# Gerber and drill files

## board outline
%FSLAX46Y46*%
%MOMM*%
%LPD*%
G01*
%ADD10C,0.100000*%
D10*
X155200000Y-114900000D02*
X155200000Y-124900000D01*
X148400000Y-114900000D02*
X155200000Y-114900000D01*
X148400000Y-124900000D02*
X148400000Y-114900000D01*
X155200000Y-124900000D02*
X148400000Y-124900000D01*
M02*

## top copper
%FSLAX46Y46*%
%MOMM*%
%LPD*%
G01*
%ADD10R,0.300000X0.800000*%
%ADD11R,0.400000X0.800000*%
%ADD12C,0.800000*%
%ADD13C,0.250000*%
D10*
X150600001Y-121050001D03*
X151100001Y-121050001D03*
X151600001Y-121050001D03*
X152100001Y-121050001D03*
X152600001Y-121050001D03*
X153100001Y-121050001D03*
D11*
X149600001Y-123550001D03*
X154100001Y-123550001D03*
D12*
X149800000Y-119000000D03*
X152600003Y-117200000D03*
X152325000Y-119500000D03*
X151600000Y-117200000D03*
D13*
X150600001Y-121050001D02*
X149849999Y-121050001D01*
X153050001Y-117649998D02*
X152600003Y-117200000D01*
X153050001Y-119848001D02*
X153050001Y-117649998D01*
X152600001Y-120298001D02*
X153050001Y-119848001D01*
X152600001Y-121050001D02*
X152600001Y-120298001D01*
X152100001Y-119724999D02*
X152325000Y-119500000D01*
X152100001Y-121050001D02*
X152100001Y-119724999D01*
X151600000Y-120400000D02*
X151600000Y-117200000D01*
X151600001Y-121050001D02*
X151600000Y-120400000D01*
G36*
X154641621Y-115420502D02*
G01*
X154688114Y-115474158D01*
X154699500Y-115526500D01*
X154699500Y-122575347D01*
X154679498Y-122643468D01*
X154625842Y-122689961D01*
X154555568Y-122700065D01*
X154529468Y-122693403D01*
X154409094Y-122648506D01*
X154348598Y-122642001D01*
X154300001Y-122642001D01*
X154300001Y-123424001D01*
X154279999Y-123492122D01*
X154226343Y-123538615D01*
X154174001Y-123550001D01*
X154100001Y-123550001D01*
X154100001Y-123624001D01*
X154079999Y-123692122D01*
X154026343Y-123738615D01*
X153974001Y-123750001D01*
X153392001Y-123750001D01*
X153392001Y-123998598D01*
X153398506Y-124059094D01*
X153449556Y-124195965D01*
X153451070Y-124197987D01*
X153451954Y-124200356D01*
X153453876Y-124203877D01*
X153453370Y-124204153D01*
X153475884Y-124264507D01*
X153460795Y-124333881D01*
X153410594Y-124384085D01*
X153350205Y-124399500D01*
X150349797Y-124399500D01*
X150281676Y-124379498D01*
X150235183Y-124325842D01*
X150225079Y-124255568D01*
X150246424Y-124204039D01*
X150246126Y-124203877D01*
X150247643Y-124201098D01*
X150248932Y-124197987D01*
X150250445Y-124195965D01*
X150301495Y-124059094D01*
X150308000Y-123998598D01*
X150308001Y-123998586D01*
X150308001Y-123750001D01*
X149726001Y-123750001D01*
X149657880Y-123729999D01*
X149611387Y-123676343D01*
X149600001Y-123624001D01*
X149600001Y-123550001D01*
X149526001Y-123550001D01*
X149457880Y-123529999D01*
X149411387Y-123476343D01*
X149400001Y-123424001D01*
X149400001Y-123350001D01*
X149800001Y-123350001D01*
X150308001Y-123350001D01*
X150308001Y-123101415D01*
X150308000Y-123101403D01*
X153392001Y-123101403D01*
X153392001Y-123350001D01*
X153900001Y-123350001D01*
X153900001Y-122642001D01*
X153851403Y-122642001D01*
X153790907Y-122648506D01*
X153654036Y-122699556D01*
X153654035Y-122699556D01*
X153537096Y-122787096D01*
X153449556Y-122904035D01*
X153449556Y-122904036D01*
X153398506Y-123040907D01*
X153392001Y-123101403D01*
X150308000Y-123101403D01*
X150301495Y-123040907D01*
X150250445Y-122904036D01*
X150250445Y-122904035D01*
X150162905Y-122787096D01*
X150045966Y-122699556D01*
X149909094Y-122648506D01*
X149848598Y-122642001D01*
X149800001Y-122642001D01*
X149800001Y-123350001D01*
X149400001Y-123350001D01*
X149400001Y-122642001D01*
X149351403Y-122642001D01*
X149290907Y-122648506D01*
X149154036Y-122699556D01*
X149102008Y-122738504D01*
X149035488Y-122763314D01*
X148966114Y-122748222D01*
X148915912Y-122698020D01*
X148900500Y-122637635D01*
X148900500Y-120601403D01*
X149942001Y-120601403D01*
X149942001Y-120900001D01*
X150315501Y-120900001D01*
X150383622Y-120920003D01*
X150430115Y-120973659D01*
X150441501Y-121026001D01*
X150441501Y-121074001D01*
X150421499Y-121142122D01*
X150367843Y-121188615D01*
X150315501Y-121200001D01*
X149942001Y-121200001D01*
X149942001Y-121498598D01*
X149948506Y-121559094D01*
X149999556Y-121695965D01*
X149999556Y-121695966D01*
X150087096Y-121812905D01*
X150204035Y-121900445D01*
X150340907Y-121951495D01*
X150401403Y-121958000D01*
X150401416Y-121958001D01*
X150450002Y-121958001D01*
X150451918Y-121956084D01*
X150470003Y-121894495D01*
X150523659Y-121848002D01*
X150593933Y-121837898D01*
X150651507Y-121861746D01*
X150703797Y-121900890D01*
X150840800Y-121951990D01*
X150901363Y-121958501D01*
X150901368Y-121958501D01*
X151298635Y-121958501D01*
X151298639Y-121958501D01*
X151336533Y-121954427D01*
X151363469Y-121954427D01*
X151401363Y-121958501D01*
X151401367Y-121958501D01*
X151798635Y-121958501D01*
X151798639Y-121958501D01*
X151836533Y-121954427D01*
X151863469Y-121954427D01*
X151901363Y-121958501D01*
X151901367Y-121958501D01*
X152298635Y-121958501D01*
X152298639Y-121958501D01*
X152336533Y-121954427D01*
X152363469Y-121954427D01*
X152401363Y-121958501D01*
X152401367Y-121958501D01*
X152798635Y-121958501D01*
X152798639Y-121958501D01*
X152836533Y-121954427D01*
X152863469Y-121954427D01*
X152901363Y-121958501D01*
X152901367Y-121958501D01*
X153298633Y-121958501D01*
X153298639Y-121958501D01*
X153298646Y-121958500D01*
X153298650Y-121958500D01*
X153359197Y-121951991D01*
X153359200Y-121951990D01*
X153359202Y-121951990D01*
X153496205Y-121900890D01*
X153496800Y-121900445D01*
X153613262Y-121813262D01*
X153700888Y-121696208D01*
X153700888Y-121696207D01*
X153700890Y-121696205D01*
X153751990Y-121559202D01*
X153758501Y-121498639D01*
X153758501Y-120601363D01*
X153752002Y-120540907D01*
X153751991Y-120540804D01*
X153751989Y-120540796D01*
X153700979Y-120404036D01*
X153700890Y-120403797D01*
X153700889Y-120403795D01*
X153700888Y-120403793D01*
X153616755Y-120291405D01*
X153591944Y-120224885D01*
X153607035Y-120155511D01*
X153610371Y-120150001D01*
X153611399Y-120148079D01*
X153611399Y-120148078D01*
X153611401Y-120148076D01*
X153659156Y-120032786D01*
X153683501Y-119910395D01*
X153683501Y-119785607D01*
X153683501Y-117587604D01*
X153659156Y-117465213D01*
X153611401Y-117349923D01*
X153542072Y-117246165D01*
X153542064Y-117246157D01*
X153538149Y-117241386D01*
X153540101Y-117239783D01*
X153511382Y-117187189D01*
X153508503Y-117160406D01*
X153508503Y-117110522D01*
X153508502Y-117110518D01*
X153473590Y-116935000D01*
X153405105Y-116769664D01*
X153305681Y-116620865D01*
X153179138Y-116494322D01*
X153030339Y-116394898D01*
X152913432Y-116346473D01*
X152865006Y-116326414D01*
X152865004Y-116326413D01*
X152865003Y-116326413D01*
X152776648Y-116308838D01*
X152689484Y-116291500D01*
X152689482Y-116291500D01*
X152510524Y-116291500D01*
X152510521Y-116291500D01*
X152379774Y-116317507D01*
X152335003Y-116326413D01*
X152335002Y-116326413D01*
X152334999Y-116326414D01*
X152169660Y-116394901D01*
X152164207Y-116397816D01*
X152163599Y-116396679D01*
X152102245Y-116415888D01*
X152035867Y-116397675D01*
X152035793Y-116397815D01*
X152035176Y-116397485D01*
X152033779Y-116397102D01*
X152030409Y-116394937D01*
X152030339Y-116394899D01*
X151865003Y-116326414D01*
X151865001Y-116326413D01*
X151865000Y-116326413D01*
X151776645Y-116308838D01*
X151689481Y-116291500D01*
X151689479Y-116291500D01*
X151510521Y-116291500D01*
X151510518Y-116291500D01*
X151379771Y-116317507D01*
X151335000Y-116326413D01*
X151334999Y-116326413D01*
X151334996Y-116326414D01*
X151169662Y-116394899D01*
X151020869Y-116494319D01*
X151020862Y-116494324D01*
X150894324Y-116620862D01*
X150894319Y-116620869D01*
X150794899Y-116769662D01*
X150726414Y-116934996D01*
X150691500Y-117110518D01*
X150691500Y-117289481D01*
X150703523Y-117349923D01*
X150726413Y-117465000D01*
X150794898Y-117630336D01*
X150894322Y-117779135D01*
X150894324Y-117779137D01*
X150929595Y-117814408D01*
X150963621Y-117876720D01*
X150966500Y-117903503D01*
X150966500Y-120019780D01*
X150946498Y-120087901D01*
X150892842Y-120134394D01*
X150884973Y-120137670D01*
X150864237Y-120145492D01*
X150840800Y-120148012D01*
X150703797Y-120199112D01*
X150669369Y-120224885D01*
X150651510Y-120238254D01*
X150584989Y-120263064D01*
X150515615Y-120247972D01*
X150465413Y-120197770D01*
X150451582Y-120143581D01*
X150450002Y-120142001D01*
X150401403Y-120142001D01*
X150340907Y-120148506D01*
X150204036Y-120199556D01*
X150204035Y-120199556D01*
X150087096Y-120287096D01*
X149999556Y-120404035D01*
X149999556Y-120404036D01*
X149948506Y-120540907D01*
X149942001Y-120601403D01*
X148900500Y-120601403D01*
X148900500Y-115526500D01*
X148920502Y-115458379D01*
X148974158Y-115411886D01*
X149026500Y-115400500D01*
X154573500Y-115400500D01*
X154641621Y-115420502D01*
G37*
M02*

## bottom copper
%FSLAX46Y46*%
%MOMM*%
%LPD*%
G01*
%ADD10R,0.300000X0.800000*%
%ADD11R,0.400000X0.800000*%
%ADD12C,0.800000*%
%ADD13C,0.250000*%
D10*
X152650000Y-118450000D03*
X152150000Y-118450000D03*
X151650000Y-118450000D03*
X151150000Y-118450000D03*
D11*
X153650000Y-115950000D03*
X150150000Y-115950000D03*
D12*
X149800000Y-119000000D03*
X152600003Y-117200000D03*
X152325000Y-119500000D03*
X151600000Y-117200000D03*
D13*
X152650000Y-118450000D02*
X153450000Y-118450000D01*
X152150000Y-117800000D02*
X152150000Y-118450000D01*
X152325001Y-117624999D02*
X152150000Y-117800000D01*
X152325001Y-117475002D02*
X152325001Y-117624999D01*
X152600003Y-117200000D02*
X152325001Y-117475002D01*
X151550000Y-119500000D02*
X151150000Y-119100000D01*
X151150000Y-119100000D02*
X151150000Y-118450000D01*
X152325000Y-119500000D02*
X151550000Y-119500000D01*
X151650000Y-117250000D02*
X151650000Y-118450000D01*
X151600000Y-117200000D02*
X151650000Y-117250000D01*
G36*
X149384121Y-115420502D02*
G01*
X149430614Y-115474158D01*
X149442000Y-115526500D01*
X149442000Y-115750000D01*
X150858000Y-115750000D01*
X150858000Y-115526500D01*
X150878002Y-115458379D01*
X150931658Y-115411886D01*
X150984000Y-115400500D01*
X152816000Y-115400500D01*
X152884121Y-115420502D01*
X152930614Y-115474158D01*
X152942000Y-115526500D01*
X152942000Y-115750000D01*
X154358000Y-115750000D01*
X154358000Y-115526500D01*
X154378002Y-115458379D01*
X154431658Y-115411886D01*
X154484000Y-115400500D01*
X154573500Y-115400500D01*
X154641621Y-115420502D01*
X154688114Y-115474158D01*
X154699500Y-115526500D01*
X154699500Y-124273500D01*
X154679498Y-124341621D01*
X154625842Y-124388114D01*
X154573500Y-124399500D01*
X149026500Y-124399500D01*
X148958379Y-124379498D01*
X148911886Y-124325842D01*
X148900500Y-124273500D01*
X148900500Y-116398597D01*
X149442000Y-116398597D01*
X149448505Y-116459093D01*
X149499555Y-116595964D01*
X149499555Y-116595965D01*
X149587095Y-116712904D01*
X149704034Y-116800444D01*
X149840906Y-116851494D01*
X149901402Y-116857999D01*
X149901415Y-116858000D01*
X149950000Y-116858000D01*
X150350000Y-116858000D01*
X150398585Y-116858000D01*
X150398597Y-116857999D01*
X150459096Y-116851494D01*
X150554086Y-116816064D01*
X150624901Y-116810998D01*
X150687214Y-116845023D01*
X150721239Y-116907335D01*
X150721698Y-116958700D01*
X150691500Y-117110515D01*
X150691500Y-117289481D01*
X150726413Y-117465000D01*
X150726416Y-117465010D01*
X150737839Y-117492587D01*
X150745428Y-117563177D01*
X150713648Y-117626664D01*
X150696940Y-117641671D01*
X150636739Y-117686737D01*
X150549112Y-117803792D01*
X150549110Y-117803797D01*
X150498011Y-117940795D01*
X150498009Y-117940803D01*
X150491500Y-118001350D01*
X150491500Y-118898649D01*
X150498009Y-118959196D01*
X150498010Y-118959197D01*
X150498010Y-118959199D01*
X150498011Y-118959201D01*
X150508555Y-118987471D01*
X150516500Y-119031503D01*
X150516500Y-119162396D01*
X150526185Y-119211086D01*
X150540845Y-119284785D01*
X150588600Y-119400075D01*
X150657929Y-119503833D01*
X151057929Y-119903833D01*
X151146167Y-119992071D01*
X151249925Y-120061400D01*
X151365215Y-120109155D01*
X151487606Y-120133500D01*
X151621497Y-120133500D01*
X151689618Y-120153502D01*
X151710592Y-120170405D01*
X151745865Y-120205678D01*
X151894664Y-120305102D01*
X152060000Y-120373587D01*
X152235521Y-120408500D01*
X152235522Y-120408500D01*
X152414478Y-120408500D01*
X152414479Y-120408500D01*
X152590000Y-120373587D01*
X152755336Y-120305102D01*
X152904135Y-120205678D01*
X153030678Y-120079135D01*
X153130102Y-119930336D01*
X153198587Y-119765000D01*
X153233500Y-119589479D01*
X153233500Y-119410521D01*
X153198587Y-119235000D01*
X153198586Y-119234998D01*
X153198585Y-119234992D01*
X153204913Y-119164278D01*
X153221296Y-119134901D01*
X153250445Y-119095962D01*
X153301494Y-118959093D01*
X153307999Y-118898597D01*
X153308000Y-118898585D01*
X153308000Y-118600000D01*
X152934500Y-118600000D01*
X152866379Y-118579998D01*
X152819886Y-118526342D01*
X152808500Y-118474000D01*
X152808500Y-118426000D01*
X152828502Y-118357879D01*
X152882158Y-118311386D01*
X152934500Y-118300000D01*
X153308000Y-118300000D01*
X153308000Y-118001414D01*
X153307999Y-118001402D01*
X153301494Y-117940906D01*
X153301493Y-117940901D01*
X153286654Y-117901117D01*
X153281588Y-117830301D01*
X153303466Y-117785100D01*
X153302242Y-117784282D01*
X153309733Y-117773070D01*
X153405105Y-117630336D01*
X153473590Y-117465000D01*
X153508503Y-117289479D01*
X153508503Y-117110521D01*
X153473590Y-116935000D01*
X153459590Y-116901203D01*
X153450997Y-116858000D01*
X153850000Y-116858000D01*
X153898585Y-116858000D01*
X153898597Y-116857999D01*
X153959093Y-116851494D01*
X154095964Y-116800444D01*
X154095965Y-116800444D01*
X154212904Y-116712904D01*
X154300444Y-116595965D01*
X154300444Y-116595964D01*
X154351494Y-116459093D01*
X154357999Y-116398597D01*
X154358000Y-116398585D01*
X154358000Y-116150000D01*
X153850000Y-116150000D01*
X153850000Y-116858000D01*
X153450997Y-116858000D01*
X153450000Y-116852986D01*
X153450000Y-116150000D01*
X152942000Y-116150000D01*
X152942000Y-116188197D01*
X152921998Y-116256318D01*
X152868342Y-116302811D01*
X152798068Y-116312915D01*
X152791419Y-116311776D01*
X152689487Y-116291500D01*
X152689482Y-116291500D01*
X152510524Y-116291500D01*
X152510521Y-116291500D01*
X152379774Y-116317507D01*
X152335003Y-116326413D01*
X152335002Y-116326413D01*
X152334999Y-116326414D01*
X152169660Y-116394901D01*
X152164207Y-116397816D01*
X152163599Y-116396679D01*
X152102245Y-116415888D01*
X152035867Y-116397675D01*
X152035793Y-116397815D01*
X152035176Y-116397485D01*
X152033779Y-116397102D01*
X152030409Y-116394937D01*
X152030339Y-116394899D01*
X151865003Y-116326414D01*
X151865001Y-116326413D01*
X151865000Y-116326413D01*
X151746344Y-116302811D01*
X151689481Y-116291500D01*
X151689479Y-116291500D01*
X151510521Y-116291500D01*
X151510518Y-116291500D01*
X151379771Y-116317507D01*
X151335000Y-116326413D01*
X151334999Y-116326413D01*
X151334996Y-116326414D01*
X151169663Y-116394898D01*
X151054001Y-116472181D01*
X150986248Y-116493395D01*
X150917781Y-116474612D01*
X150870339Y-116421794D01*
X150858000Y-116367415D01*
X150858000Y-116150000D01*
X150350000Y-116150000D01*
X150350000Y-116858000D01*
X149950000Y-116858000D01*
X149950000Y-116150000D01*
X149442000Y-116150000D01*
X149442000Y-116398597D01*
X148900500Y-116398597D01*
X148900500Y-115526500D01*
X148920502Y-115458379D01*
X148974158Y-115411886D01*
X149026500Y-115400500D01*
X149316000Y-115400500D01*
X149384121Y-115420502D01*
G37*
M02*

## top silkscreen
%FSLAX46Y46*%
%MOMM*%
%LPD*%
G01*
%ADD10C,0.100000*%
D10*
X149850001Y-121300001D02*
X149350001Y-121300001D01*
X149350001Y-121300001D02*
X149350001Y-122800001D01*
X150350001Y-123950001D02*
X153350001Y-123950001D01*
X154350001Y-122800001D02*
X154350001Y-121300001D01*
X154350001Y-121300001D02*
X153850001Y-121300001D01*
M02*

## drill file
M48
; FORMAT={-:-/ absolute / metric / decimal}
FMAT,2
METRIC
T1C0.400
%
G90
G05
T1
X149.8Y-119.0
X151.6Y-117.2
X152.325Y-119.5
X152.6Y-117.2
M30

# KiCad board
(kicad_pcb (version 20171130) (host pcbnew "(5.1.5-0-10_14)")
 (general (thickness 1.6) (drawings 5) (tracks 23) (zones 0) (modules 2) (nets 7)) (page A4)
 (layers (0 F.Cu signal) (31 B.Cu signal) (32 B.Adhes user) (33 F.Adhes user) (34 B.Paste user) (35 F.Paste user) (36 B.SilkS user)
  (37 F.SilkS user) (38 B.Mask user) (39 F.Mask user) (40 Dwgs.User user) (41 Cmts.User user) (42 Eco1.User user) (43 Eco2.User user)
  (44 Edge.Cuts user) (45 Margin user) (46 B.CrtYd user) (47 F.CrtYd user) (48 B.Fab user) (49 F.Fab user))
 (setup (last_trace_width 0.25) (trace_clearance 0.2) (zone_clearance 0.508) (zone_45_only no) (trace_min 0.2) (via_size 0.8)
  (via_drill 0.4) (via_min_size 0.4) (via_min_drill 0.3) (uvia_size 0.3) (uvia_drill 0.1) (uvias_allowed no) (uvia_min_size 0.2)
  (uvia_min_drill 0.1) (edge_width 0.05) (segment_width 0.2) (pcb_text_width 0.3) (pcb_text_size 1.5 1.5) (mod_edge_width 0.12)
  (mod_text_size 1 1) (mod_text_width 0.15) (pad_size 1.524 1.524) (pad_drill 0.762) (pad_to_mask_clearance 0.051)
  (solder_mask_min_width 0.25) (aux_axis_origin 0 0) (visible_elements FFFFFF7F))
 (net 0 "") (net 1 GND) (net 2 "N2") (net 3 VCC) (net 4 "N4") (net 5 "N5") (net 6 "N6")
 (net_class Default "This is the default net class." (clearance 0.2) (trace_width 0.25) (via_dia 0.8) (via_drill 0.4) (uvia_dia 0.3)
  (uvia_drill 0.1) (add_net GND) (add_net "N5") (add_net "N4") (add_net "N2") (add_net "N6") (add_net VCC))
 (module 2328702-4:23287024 (layer B.Cu) (at 151.9 117)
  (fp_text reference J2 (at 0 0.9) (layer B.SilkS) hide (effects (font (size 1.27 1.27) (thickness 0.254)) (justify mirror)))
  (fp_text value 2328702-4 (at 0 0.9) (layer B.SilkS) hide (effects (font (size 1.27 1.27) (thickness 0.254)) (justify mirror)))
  (pad 1 smd rect (at 0.75 1.45) (size 0.3 0.8) (layers B.Cu B.Paste B.Mask) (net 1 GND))
  (pad 2 smd rect (at 0.25 1.45) (size 0.3 0.8) (layers B.Cu B.Paste B.Mask) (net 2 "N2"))
  (pad 3 smd rect (at -0.25 1.45) (size 0.3 0.8) (layers B.Cu B.Paste B.Mask) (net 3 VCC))
  (pad 4 smd rect (at -0.75 1.45) (size 0.3 0.8) (layers B.Cu B.Paste B.Mask) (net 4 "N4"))
  (pad MP1 smd rect (at 1.75 -1.05) (size 0.4 0.8) (layers B.Cu B.Paste B.Mask) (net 1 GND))
  (pad MP2 smd rect (at -1.75 -1.05) (size 0.4 0.8) (layers B.Cu B.Paste B.Mask) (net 1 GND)))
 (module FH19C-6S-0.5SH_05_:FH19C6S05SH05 (layer F.Cu) (at 151.850001 122.500001)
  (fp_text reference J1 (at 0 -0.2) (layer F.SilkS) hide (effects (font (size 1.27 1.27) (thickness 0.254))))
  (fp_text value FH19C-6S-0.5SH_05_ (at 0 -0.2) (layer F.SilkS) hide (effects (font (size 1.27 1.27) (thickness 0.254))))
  (fp_line (start -2 -1.2) (end -2.5 -1.2) (layer F.SilkS) (width 0.1))
  (fp_line (start -2.5 -1.2) (end -2.5 0.3) (layer F.SilkS) (width 0.1))
  (fp_line (start -1.5 1.45) (end 1.5 1.45) (layer F.SilkS) (width 0.1))
  (fp_line (start 2.5 0.3) (end 2.5 -1.2) (layer F.SilkS) (width 0.1))
  (fp_line (start 2.5 -1.2) (end 2 -1.2) (layer F.SilkS) (width 0.1))
  (pad 1 smd rect (at -1.25 -1.45) (size 0.3 0.8) (layers F.Cu F.Paste F.Mask) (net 1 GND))
  (pad 2 smd rect (at -0.75 -1.45) (size 0.3 0.8) (layers F.Cu F.Paste F.Mask) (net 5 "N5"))
  (pad 3 smd rect (at -0.25 -1.45) (size 0.3 0.8) (layers F.Cu F.Paste F.Mask) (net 3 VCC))
  (pad 4 smd rect (at 0.25 -1.45) (size 0.3 0.8) (layers F.Cu F.Paste F.Mask) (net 4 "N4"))
  (pad 5 smd rect (at 0.75 -1.45) (size 0.3 0.8) (layers F.Cu F.Paste F.Mask) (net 2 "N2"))
  (pad 6 smd rect (at 1.25 -1.45) (size 0.3 0.8) (layers F.Cu F.Paste F.Mask) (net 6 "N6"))
  (pad 7 smd rect (at -2.25 1.05) (size 0.4 0.8) (layers F.Cu F.Paste F.Mask) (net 1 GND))
  (pad 8 smd rect (at 2.25 1.05) (size 0.4 0.8) (layers F.Cu F.Paste F.Mask) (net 1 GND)))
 (gr_line (start 155.2 114.9) (end 155.2 124.9) (layer Edge.Cuts) (width 0.1))
 (gr_line (start 148.4 114.9) (end 155.2 114.9) (layer Edge.Cuts) (width 0.1))
 (gr_line (start 148.4 124.9) (end 148.4 114.9) (layer Edge.Cuts) (width 0.1))
 (gr_line (start 155.2 124.9) (end 148.4 124.9) (layer Edge.Cuts) (width 0.1))
 (segment (start 150.600001 121.050001) (end 149.849999 121.050001) (width 0.25) (layer F.Cu) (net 1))
 (segment (start 152.65 118.45) (end 153.45 118.45) (width 0.25) (layer B.Cu) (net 1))
 (via (at 149.8 119) (size 0.8) (drill 0.4) (layers F.Cu B.Cu) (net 1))
 (via (at 152.600003 117.2) (size 0.8) (drill 0.4) (layers F.Cu B.Cu) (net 2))
 (segment (start 153.050001 117.649998) (end 152.600003 117.2) (width 0.25) (layer F.Cu) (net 2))
 (segment (start 153.050001 119.848001) (end 153.050001 117.649998) (width 0.25) (layer F.Cu) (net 2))
 (segment (start 152.600001 120.298001) (end 153.050001 119.848001) (width 0.25) (layer F.Cu) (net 2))
 (segment (start 152.600001 121.050001) (end 152.600001 120.298001) (width 0.25) (layer F.Cu) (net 2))
 (segment (start 152.15 117.8) (end 152.15 118.45) (width 0.25) (layer B.Cu) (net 2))
 (segment (start 152.325001 117.624999) (end 152.15 117.8) (width 0.25) (layer B.Cu) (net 2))
 (segment (start 152.325001 117.475002) (end 152.325001 117.624999) (width 0.25) (layer B.Cu) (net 2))
 (segment (start 152.600003 117.2) (end 152.325001 117.475002) (width 0.25) (layer B.Cu) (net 2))
 (via (at 152.325 119.5) (size 0.8) (drill 0.4) (layers F.Cu B.Cu) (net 4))
 (segment (start 152.100001 119.724999) (end 152.325 119.5) (width 0.25) (layer F.Cu) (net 4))
 (segment (start 152.100001 121.050001) (end 152.100001 119.724999) (width 0.25) (layer F.Cu) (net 4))
 (segment (start 151.55 119.5) (end 151.15 119.1) (width 0.25) (layer B.Cu) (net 4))
 (segment (start 151.15 119.1) (end 151.15 118.45) (width 0.25) (layer B.Cu) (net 4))
 (segment (start 152.325 119.5) (end 151.55 119.5) (width 0.25) (layer B.Cu) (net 4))
 (via (at 151.6 117.2) (size 0.8) (drill 0.4) (layers F.Cu B.Cu) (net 3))
 (segment (start 151.6 120.4) (end 151.6 117.2) (width 0.25) (layer F.Cu) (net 3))
 (segment (start 151.600001 121.050001) (end 151.6 120.4) (width 0.25) (layer F.Cu) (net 3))
 (segment (start 151.65 117.25) (end 151.65 118.45) (width 0.25) (layer B.Cu) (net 3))
 (segment (start 151.6 117.2) (end 151.65 117.25) (width 0.25) (layer B.Cu) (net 3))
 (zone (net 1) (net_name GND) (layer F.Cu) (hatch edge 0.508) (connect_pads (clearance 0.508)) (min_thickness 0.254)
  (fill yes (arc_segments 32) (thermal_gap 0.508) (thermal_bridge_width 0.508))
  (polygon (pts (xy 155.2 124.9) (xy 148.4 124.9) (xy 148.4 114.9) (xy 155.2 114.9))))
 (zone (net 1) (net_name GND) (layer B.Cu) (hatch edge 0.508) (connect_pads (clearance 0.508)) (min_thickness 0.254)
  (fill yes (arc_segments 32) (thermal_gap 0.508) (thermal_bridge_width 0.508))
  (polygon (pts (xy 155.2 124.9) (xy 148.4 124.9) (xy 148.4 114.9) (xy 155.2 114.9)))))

